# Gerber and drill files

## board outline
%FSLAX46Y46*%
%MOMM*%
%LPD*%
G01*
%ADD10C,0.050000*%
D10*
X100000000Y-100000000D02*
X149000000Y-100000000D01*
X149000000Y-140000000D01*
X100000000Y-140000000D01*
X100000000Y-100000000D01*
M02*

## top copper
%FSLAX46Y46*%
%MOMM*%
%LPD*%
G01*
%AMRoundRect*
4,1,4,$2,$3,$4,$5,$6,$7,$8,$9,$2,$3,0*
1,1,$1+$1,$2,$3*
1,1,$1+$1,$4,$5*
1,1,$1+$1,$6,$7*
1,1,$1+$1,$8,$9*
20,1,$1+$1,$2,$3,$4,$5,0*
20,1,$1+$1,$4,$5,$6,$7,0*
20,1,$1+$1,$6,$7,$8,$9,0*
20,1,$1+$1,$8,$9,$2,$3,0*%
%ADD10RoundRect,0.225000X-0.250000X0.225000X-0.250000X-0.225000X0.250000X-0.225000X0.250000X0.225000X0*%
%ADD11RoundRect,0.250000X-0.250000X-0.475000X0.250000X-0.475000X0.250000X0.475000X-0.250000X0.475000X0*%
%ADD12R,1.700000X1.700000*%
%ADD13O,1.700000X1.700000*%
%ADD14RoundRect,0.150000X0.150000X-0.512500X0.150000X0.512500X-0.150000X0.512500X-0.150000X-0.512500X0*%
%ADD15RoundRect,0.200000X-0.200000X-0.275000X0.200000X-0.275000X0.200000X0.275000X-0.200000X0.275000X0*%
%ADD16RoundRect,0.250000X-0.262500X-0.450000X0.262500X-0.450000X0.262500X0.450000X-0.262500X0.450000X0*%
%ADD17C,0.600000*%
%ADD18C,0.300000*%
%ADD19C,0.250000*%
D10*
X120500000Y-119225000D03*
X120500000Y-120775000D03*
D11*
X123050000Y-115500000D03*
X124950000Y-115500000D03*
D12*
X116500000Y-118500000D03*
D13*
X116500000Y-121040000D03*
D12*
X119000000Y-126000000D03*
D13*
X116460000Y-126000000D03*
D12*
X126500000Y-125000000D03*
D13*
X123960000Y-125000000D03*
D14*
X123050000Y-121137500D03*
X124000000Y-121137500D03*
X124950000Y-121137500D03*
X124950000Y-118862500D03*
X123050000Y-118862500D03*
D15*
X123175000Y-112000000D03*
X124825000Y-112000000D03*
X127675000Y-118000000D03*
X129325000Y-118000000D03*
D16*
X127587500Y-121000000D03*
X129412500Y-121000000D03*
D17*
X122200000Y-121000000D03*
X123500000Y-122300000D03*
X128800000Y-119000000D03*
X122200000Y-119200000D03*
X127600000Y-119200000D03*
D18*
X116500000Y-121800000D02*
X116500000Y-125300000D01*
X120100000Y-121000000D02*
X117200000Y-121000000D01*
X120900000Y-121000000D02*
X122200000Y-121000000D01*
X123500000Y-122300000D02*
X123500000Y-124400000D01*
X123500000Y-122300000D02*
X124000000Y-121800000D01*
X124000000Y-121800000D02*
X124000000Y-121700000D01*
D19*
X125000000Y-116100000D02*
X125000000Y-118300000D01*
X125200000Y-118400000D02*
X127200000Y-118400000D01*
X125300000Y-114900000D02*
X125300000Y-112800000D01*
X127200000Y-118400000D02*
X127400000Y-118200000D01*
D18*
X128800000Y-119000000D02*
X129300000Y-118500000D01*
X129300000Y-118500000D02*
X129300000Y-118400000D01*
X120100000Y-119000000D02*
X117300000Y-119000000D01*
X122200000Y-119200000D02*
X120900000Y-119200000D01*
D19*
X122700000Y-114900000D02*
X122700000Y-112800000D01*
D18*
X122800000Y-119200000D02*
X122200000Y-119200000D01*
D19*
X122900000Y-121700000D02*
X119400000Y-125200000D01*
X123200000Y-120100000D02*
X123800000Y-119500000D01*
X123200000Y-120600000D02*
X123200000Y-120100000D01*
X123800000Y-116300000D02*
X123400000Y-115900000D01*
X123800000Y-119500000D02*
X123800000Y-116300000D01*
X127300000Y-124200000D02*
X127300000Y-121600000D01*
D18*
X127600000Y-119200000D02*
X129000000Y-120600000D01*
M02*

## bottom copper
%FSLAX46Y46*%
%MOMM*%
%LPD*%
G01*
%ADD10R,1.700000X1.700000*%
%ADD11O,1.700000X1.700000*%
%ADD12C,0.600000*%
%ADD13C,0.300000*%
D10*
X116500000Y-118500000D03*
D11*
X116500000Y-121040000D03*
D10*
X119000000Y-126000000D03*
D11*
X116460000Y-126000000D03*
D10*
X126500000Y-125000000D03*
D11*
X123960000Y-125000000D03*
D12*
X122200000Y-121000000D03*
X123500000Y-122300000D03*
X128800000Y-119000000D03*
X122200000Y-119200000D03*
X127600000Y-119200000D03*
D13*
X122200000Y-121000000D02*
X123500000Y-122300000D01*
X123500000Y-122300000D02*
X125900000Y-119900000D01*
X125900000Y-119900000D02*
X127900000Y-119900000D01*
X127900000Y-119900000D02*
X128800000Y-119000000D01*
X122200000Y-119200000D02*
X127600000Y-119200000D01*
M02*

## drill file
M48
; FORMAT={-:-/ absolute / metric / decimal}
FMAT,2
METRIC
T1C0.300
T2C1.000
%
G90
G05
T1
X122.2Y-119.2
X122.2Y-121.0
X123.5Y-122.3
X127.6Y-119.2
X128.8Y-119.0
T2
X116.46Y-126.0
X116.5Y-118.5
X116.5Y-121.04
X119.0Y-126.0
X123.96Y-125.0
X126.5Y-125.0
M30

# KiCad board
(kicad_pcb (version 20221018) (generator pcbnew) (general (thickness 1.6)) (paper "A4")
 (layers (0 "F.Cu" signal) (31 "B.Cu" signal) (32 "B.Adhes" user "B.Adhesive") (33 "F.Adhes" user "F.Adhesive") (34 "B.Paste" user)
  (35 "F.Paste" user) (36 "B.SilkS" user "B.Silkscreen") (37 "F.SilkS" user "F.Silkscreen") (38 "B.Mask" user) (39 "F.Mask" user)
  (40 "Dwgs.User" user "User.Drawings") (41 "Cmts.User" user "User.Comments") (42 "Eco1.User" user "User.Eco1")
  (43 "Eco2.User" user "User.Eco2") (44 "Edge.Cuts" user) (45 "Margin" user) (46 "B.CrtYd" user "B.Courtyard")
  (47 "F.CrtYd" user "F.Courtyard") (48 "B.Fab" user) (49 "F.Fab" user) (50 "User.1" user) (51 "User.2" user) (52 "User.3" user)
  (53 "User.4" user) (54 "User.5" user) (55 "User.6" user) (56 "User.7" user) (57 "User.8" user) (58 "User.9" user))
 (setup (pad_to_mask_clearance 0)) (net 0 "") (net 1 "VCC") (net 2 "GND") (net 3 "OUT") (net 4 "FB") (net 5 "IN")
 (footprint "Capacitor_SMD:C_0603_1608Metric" (layer "F.Cu") (at 120.5 120 -90)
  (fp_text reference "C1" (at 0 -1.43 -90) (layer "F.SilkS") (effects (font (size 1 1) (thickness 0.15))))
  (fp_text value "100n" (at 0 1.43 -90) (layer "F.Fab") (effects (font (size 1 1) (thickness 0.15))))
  (pad "1" smd roundrect (at -0.775 0 270) (size 0.9 0.95) (layers "F.Cu" "F.Paste" "F.Mask") (roundrect_rratio 0.25) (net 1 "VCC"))
  (pad "2" smd roundrect (at 0.775 0 270) (size 0.9 0.95) (layers "F.Cu" "F.Paste" "F.Mask") (roundrect_rratio 0.25) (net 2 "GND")))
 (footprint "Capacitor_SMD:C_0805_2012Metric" (layer "F.Cu") (at 124 115.5)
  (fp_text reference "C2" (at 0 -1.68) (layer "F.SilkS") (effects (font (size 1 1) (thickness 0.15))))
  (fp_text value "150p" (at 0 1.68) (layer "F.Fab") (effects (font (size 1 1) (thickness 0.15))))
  (pad "1" smd roundrect (at -0.95 0) (size 1 1.45) (layers "F.Cu" "F.Paste" "F.Mask") (roundrect_rratio 0.25) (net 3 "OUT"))
  (pad "2" smd roundrect (at 0.95 0) (size 1 1.45) (layers "F.Cu" "F.Paste" "F.Mask") (roundrect_rratio 0.25) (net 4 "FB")))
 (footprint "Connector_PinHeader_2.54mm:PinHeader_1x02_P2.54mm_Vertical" (layer "F.Cu") (at 116.5 118.5)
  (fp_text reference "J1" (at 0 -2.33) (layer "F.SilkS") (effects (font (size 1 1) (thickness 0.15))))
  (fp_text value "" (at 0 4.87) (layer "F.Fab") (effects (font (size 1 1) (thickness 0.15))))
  (pad "1" thru_hole rect (at 0 0) (size 1.7 1.7) (drill 1) (layers "*.Cu" "*.Mask") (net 1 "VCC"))
  (pad "2" thru_hole oval (at 0 2.54) (size 1.7 1.7) (drill 1) (layers "*.Cu" "*.Mask") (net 2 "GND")))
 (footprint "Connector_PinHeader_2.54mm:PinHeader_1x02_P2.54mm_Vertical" (layer "F.Cu") (at 119 126 -90)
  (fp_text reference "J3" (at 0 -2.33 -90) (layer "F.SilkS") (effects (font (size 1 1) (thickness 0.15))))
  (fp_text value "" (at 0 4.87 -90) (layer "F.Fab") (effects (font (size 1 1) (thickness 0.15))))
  (pad "1" thru_hole rect (at 0 0 270) (size 1.7 1.7) (drill 1) (layers "*.Cu" "*.Mask") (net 3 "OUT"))
  (pad "2" thru_hole oval (at 0 2.54 270) (size 1.7 1.7) (drill 1) (layers "*.Cu" "*.Mask") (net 2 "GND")))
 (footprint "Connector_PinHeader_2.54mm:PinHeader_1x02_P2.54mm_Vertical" (layer "F.Cu") (at 126.5 125 -90)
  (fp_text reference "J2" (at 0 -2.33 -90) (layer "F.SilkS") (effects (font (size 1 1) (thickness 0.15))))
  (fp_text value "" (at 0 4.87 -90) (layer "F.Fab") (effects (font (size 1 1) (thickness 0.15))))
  (pad "1" thru_hole rect (at 0 0 270) (size 1.7 1.7) (drill 1) (layers "*.Cu" "*.Mask") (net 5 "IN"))
  (pad "2" thru_hole oval (at 0 2.54 270) (size 1.7 1.7) (drill 1) (layers "*.Cu" "*.Mask") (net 2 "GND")))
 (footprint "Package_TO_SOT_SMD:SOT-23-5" (layer "F.Cu") (at 124 120 90)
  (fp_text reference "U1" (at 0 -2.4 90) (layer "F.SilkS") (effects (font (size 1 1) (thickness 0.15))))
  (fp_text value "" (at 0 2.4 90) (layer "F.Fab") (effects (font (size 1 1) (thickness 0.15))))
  (pad "1" smd roundrect (at -1.1375 -0.95 90) (size 1.325 0.6) (layers "F.Cu" "F.Paste" "F.Mask") (roundrect_rratio 0.25) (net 3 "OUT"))
  (pad "2" smd roundrect (at -1.1375 0 90) (size 1.325 0.6) (layers "F.Cu" "F.Paste" "F.Mask") (roundrect_rratio 0.25) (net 2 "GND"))
  (pad "3" smd roundrect (at -1.1375 0.95 90) (size 1.325 0.6) (layers "F.Cu" "F.Paste" "F.Mask") (roundrect_rratio 0.25))
  (pad "4" smd roundrect (at 1.1375 0.95 90) (size 1.325 0.6) (layers "F.Cu" "F.Paste" "F.Mask") (roundrect_rratio 0.25) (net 4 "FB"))
  (pad "5" smd roundrect (at 1.1375 -0.95 90) (size 1.325 0.6) (layers "F.Cu" "F.Paste" "F.Mask") (roundrect_rratio 0.25) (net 1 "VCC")))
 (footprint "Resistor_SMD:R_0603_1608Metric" (layer "F.Cu") (at 124 112)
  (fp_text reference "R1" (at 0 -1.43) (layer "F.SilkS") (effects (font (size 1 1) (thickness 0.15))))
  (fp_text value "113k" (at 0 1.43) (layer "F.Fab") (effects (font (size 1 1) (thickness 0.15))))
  (pad "1" smd roundrect (at -0.825 0) (size 0.8 0.95) (layers "F.Cu" "F.Paste" "F.Mask") (roundrect_rratio 0.25) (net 3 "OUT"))
  (pad "2" smd roundrect (at 0.825 0) (size 0.8 0.95) (layers "F.Cu" "F.Paste" "F.Mask") (roundrect_rratio 0.25) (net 4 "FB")))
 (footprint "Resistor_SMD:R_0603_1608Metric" (layer "F.Cu") (at 128.5 118)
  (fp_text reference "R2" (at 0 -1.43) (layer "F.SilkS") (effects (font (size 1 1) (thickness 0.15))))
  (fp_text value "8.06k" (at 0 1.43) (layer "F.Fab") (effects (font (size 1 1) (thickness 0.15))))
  (pad "1" smd roundrect (at -0.825 0) (size 0.8 0.95) (layers "F.Cu" "F.Paste" "F.Mask") (roundrect_rratio 0.25) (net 4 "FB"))
  (pad "2" smd roundrect (at 0.825 0) (size 0.8 0.95) (layers "F.Cu" "F.Paste" "F.Mask") (roundrect_rratio 0.25) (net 2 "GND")))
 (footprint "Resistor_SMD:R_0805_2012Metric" (layer "F.Cu") (at 128.5 121)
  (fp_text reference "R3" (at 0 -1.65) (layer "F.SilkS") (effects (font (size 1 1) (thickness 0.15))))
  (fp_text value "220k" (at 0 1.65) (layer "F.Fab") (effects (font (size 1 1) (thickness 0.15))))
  (pad "1" smd roundrect (at -0.9125 0) (size 1.025 1.4) (layers "F.Cu" "F.Paste" "F.Mask") (roundrect_rratio 0.243902) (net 5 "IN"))
  (pad "2" smd roundrect (at 0.9125 0) (size 1.025 1.4) (layers "F.Cu" "F.Paste" "F.Mask") (roundrect_rratio 0.243902) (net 1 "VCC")))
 (gr_rect (start 100 100) (end 149 140) (stroke (width 0.05) (type default)) (fill none) (layer "Edge.Cuts"))
 (segment (start 116.5 121.8) (end 116.5 125.3) (width 0.3) (layer "F.Cu") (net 2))
 (segment (start 120.1 121) (end 117.2 121) (width 0.3) (layer "F.Cu") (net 2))
 (segment (start 120.9 121) (end 122.2 121) (width 0.3) (layer "F.Cu") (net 2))
 (segment (start 123.5 122.3) (end 123.5 124.4) (width 0.3) (layer "F.Cu") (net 2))
 (segment (start 123.5 122.3) (end 124 121.8) (width 0.3) (layer "F.Cu") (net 2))
 (segment (start 124 121.8) (end 124 121.7) (width 0.3) (layer "F.Cu") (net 2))
 (segment (start 125 116.1) (end 125 118.3) (width 0.25) (layer "F.Cu") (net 4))
 (segment (start 125.2 118.4) (end 127.2 118.4) (width 0.25) (layer "F.Cu") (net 4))
 (segment (start 125.3 114.9) (end 125.3 112.8) (width 0.25) (layer "F.Cu") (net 4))
 (segment (start 127.2 118.4) (end 127.4 118.2) (width 0.25) (layer "F.Cu") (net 4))
 (segment (start 128.8 119) (end 129.3 118.5) (width 0.3) (layer "F.Cu") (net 2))
 (segment (start 129.3 118.5) (end 129.3 118.4) (width 0.3) (layer "F.Cu") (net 2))
 (via (at 122.2 121) (size 0.6) (drill 0.3) (layers "F.Cu" "B.Cu") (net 2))
 (via (at 123.5 122.3) (size 0.6) (drill 0.3) (layers "F.Cu" "B.Cu") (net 2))
 (via (at 128.8 119) (size 0.6) (drill 0.3) (layers "F.Cu" "B.Cu") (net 2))
 (segment (start 120.1 119) (end 117.3 119) (width 0.3) (layer "F.Cu") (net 1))
 (segment (start 122.2 119.2) (end 120.9 119.2) (width 0.3) (layer "F.Cu") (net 1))
 (segment (start 122.2 121) (end 123.5 122.3) (width 0.3) (layer "B.Cu") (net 2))
 (segment (start 122.7 114.9) (end 122.7 112.8) (width 0.25) (layer "F.Cu") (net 3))
 (segment (start 122.8 119.2) (end 122.2 119.2) (width 0.3) (layer "F.Cu") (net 1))
 (segment (start 122.9 121.7) (end 119.4 125.2) (width 0.25) (layer "F.Cu") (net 3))
 (segment (start 123.2 120.1) (end 123.8 119.5) (width 0.25) (layer "F.Cu") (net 3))
 (segment (start 123.2 120.6) (end 123.2 120.1) (width 0.25) (layer "F.Cu") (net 3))
 (segment (start 123.5 122.3) (end 125.9 119.9) (width 0.3) (layer "B.Cu") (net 2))
 (segment (start 123.8 116.3) (end 123.4 115.9) (width 0.25) (layer "F.Cu") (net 3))
 (segment (start 123.8 119.5) (end 123.8 116.3) (width 0.25) (layer "F.Cu") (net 3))
 (segment (start 125.9 119.9) (end 127.9 119.9) (width 0.3) (layer "B.Cu") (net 2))
 (segment (start 127.3 124.2) (end 127.3 121.6) (width 0.25) (layer "F.Cu") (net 5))
 (segment (start 127.6 119.2) (end 129 120.6) (width 0.3) (layer "F.Cu") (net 1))
 (segment (start 127.9 119.9) (end 128.8 119) (width 0.3) (layer "B.Cu") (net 2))
 (via (at 122.2 119.2) (size 0.6) (drill 0.3) (layers "F.Cu" "B.Cu") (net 1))
 (via (at 127.6 119.2) (size 0.6) (drill 0.3) (layers "F.Cu" "B.Cu") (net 1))
 (segment (start 122.2 119.2) (end 127.6 119.2) (width 0.3) (layer "B.Cu") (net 1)))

